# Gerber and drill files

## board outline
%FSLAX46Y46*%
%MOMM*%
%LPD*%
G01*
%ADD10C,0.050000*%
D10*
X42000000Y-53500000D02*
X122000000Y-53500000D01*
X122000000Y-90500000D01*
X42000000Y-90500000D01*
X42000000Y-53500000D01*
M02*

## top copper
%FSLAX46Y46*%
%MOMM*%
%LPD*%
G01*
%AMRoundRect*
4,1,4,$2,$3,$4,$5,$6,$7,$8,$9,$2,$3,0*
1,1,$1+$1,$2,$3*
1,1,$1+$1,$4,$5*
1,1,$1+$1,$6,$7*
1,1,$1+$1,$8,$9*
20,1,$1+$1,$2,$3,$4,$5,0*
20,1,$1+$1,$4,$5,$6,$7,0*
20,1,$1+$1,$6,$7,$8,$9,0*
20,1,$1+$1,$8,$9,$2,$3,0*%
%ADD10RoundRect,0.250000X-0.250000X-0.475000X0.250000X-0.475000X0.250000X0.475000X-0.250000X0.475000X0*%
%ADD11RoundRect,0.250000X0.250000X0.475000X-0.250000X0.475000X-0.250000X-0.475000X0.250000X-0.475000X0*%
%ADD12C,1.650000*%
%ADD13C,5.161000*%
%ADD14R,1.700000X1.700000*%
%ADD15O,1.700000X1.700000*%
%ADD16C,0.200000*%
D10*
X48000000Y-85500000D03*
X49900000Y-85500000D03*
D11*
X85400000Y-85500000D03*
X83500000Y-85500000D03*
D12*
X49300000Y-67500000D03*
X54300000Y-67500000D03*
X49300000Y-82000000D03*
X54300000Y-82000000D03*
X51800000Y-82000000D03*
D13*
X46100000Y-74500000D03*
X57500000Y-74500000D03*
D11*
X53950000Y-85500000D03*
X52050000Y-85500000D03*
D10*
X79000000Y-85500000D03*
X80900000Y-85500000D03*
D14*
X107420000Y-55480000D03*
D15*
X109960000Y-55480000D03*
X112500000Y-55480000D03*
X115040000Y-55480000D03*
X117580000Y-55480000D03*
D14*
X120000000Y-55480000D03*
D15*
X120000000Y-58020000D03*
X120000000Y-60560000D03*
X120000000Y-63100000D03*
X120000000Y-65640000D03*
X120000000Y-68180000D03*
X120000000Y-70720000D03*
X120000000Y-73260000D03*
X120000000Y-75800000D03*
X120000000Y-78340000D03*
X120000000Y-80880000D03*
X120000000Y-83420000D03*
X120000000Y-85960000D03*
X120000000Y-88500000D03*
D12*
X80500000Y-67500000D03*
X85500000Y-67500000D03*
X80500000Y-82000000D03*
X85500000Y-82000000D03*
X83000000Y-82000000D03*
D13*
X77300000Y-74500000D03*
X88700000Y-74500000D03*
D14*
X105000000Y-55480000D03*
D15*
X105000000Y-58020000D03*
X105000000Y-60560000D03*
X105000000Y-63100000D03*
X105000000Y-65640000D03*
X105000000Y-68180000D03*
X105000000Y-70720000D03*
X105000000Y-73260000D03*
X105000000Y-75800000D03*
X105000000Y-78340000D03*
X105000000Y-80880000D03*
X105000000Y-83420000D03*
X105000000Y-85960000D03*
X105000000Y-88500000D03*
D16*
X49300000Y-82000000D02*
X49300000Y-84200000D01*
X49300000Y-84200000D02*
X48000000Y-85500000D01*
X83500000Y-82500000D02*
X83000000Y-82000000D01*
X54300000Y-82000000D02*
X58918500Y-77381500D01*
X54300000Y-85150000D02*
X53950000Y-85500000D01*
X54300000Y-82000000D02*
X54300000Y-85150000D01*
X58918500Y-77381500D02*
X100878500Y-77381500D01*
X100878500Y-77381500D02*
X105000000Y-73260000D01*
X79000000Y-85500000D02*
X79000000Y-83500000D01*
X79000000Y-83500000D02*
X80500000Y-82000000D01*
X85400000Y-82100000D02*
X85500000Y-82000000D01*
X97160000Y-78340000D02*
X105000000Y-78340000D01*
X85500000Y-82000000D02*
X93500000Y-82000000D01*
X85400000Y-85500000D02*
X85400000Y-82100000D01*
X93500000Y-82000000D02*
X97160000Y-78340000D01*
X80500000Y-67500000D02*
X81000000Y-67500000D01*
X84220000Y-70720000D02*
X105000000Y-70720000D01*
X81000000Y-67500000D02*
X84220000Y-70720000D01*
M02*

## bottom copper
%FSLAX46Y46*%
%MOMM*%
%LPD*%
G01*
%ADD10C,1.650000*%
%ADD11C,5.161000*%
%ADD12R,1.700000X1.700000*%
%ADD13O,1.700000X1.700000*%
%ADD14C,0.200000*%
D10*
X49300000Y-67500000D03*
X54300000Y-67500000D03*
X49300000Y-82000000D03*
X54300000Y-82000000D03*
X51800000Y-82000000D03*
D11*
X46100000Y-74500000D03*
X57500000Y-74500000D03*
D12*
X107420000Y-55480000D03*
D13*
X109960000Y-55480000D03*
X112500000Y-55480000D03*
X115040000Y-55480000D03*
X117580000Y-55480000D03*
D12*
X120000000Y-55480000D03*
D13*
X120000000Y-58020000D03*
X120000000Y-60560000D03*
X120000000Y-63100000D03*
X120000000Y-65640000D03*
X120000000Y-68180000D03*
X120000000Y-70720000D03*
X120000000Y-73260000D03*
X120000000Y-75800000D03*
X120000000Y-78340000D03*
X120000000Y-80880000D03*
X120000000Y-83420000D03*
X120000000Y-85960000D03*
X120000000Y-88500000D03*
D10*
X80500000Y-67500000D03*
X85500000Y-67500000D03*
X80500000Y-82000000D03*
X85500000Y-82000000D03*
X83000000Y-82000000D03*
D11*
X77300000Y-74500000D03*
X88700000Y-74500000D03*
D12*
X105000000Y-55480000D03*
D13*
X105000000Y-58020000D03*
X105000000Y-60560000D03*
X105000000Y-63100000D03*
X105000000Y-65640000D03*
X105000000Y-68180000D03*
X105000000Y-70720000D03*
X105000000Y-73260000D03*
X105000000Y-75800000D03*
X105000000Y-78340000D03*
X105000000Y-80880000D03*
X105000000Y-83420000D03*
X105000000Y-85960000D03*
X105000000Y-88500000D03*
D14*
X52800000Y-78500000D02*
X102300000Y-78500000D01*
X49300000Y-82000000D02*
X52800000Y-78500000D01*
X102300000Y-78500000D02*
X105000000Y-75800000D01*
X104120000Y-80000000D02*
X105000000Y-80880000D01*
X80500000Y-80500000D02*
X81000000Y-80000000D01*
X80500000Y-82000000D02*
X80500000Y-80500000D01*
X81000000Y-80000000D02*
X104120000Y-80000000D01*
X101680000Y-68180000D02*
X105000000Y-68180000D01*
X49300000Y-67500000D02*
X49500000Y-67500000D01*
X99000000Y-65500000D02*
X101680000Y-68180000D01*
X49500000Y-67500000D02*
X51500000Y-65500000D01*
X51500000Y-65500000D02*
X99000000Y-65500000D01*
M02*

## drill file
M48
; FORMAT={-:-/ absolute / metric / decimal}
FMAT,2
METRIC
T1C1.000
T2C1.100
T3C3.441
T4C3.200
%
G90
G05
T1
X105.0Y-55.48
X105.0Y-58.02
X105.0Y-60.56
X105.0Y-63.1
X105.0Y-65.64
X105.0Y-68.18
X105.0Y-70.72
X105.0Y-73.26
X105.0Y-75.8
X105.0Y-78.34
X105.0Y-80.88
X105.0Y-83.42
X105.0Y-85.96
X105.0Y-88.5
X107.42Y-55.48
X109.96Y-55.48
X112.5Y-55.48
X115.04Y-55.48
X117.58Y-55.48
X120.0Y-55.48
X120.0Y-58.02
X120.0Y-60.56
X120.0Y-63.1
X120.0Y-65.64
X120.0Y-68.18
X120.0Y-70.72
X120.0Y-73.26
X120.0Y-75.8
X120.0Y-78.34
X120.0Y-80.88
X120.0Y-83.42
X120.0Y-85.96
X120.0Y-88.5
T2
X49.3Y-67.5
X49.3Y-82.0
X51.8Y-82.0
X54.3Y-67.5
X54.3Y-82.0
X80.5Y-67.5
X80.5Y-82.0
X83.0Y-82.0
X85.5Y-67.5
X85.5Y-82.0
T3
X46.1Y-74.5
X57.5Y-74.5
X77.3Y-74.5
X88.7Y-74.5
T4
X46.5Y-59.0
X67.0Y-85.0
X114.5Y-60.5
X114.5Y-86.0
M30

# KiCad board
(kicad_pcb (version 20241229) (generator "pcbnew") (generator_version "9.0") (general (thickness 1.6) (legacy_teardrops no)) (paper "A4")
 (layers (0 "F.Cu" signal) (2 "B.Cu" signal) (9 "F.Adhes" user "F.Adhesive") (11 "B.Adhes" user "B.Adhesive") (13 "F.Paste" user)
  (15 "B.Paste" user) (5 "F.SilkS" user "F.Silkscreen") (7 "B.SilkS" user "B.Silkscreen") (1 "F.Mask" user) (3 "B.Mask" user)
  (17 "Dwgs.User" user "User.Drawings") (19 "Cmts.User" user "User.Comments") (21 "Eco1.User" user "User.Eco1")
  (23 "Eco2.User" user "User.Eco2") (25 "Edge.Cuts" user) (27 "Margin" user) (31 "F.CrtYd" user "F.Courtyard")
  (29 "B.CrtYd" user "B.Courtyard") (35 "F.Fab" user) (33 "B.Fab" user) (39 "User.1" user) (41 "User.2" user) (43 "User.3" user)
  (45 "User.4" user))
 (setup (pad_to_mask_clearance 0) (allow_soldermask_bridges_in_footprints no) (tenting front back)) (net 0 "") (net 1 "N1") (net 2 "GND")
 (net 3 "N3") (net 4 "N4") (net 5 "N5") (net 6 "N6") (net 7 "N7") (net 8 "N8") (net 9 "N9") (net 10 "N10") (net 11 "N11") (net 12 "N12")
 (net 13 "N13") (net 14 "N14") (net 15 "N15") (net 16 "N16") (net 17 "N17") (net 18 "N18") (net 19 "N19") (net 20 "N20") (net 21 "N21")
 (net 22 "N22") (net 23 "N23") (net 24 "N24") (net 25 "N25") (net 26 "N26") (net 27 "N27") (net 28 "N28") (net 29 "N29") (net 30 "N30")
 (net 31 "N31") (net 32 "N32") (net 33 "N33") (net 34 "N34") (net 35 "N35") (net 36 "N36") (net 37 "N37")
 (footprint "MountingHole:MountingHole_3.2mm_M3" (layer "F.Cu") (at 114.5 60.5)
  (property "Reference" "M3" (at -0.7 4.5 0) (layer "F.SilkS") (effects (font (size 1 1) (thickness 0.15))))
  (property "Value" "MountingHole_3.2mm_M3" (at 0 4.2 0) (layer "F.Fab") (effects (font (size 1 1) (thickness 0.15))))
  (pad "" np_thru_hole circle (at 0 0) (size 3.2 3.2) (drill 3.2) (layers "*.Cu" "*.Mask")))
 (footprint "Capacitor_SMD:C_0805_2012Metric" (layer "F.Cu") (at 48.95 85.5)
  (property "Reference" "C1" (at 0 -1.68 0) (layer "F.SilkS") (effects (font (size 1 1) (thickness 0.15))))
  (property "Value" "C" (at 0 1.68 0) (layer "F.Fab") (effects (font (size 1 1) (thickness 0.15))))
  (pad "1" smd roundrect (at -0.95 0) (size 1 1.45) (layers "F.Cu" "F.Mask" "F.Paste") (roundrect_rratio 0.25) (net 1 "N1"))
  (pad "2" smd roundrect (at 0.95 0) (size 1 1.45) (layers "F.Cu" "F.Mask" "F.Paste") (roundrect_rratio 0.25) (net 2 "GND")))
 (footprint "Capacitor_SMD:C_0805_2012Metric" (layer "F.Cu") (at 84.45 85.5 180)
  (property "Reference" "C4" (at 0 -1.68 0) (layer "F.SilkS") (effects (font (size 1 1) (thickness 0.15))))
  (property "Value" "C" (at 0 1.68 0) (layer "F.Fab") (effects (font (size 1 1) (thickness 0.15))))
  (pad "1" smd roundrect (at -0.95 0 180) (size 1 1.45) (layers "F.Cu" "F.Mask" "F.Paste") (roundrect_rratio 0.25) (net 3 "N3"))
  (pad "2" smd roundrect (at 0.95 0 180) (size 1 1.45) (layers "F.Cu" "F.Mask" "F.Paste") (roundrect_rratio 0.25) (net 2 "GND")))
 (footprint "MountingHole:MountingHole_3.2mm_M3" (layer "F.Cu") (at 46.5 59)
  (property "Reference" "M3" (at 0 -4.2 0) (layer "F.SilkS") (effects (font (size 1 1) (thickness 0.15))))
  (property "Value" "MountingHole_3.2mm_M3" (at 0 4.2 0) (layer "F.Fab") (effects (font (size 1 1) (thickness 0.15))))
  (pad "" np_thru_hole circle (at 0 0) (size 3.2 3.2) (drill 3.2) (layers "*.Cu" "*.Mask")))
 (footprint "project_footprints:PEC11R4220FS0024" (layer "F.Cu") (at 49.3 67.5)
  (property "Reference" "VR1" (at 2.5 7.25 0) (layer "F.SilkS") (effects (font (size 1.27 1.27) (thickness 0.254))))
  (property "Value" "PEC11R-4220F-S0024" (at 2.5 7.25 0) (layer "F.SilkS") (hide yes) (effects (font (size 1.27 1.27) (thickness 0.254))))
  (pad "1" thru_hole circle (at 0 0) (size 1.65 1.65) (drill 1.1) (layers "*.Cu" "*.Mask") (remove_unused_layers no) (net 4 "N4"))
  (pad "2" thru_hole circle (at 5 0) (size 1.65 1.65) (drill 1.1) (layers "*.Cu" "*.Mask") (remove_unused_layers no) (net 2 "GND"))
  (pad "A1" thru_hole circle (at 0 14.5) (size 1.65 1.65) (drill 1.1) (layers "*.Cu" "*.Mask") (remove_unused_layers no) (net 1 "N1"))
  (pad "B1" thru_hole circle (at 5 14.5) (size 1.65 1.65) (drill 1.1) (layers "*.Cu" "*.Mask") (remove_unused_layers no) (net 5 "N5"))
  (pad "C1" thru_hole circle (at 2.5 14.5) (size 1.65 1.65) (drill 1.1) (layers "*.Cu" "*.Mask") (remove_unused_layers no) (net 2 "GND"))
  (pad "MH1" thru_hole circle (at -3.2 7) (size 5.161 5.161) (drill 3.4409) (layers "*.Cu" "*.Mask") (remove_unused_layers no) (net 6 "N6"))
  (pad "MH2" thru_hole circle (at 8.2 7) (size 5.161 5.161) (drill 3.4409) (layers "*.Cu" "*.Mask") (remove_unused_layers no) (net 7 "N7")))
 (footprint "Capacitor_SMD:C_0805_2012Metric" (layer "F.Cu") (at 53 85.5 180)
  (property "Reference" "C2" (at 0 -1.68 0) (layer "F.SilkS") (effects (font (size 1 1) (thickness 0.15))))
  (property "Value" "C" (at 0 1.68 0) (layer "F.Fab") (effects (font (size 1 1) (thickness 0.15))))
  (pad "1" smd roundrect (at -0.95 0 180) (size 1 1.45) (layers "F.Cu" "F.Mask" "F.Paste") (roundrect_rratio 0.25) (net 5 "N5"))
  (pad "2" smd roundrect (at 0.95 0 180) (size 1 1.45) (layers "F.Cu" "F.Mask" "F.Paste") (roundrect_rratio 0.25) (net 2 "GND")))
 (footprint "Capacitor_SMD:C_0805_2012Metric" (layer "F.Cu") (at 79.95 85.5)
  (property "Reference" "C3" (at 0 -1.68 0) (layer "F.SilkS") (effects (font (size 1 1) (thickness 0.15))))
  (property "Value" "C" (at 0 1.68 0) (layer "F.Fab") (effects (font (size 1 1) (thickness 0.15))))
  (pad "1" smd roundrect (at -0.95 0) (size 1 1.45) (layers "F.Cu" "F.Mask" "F.Paste") (roundrect_rratio 0.25) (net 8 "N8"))
  (pad "2" smd roundrect (at 0.95 0) (size 1 1.45) (layers "F.Cu" "F.Mask" "F.Paste") (roundrect_rratio 0.25) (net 2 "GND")))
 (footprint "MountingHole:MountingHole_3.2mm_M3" (layer "F.Cu") (at 114.5 86)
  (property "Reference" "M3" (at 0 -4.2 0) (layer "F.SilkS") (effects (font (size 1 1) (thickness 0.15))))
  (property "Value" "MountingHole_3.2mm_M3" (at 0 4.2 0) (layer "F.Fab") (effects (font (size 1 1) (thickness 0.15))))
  (pad "" np_thru_hole circle (at 0 0) (size 3.2 3.2) (drill 3.2) (layers "*.Cu" "*.Mask")))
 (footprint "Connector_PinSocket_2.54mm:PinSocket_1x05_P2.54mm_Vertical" (layer "F.Cu") (at 107.42 55.48 90)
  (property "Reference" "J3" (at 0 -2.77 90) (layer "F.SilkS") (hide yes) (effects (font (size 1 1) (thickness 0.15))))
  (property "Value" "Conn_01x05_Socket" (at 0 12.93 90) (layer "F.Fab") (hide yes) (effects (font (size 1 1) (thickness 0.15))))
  (pad "1" thru_hole rect (at 0 0 90) (size 1.7 1.7) (drill 1) (layers "*.Cu" "*.Mask") (remove_unused_layers no) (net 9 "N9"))
  (pad "2" thru_hole oval (at 0 2.54 90) (size 1.7 1.7) (drill 1) (layers "*.Cu" "*.Mask") (remove_unused_layers no) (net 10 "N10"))
  (pad "3" thru_hole oval (at 0 5.08 90) (size 1.7 1.7) (drill 1) (layers "*.Cu" "*.Mask") (remove_unused_layers no) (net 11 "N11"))
  (pad "4" thru_hole oval (at 0 7.62 90) (size 1.7 1.7) (drill 1) (layers "*.Cu" "*.Mask") (remove_unused_layers no) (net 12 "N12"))
  (pad "5" thru_hole oval (at 0 10.16 90) (size 1.7 1.7) (drill 1) (layers "*.Cu" "*.Mask") (remove_unused_layers no) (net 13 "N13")))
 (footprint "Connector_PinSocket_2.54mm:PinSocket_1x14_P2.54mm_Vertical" (layer "F.Cu") (at 120 55.48)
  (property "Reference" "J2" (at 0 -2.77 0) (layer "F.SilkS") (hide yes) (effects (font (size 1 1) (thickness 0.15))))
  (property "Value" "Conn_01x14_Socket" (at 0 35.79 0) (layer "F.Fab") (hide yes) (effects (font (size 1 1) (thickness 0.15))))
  (pad "1" thru_hole rect (at 0 0) (size 1.7 1.7) (drill 1) (layers "*.Cu" "*.Mask") (remove_unused_layers no) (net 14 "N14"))
  (pad "2" thru_hole oval (at 0 2.54) (size 1.7 1.7) (drill 1) (layers "*.Cu" "*.Mask") (remove_unused_layers no) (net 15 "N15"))
  (pad "3" thru_hole oval (at 0 5.08) (size 1.7 1.7) (drill 1) (layers "*.Cu" "*.Mask") (remove_unused_layers no) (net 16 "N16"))
  (pad "4" thru_hole oval (at 0 7.62) (size 1.7 1.7) (drill 1) (layers "*.Cu" "*.Mask") (remove_unused_layers no) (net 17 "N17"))
  (pad "5" thru_hole oval (at 0 10.16) (size 1.7 1.7) (drill 1) (layers "*.Cu" "*.Mask") (remove_unused_layers no) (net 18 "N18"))
  (pad "6" thru_hole oval (at 0 12.7) (size 1.7 1.7) (drill 1) (layers "*.Cu" "*.Mask") (remove_unused_layers no) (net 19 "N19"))
  (pad "7" thru_hole oval (at 0 15.24) (size 1.7 1.7) (drill 1) (layers "*.Cu" "*.Mask") (remove_unused_layers no) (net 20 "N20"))
  (pad "8" thru_hole oval (at 0 17.78) (size 1.7 1.7) (drill 1) (layers "*.Cu" "*.Mask") (remove_unused_layers no) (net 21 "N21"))
  (pad "9" thru_hole oval (at 0 20.32) (size 1.7 1.7) (drill 1) (layers "*.Cu" "*.Mask") (remove_unused_layers no) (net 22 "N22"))
  (pad "10" thru_hole oval (at 0 22.86) (size 1.7 1.7) (drill 1) (layers "*.Cu" "*.Mask") (remove_unused_layers no) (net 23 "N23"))
  (pad "11" thru_hole oval (at 0 25.4) (size 1.7 1.7) (drill 1) (layers "*.Cu" "*.Mask") (remove_unused_layers no) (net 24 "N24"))
  (pad "12" thru_hole oval (at 0 27.94) (size 1.7 1.7) (drill 1) (layers "*.Cu" "*.Mask") (remove_unused_layers no) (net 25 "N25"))
  (pad "13" thru_hole oval (at 0 30.48) (size 1.7 1.7) (drill 1) (layers "*.Cu" "*.Mask") (remove_unused_layers no) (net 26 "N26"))
  (pad "14" thru_hole oval (at 0 33.02) (size 1.7 1.7) (drill 1) (layers "*.Cu" "*.Mask") (remove_unused_layers no) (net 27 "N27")))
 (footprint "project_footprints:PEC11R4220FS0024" (layer "F.Cu") (at 80.5 67.5)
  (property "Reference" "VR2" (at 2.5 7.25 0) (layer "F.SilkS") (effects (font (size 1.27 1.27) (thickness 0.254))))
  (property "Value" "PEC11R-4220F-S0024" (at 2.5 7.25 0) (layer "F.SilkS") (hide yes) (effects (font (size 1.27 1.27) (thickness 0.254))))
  (pad "1" thru_hole circle (at 0 0) (size 1.65 1.65) (drill 1.1) (layers "*.Cu" "*.Mask") (remove_unused_layers no) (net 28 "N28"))
  (pad "2" thru_hole circle (at 5 0) (size 1.65 1.65) (drill 1.1) (layers "*.Cu" "*.Mask") (remove_unused_layers no) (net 2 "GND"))
  (pad "A1" thru_hole circle (at 0 14.5) (size 1.65 1.65) (drill 1.1) (layers "*.Cu" "*.Mask") (remove_unused_layers no) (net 8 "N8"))
  (pad "B1" thru_hole circle (at 5 14.5) (size 1.65 1.65) (drill 1.1) (layers "*.Cu" "*.Mask") (remove_unused_layers no) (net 3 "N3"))
  (pad "C1" thru_hole circle (at 2.5 14.5) (size 1.65 1.65) (drill 1.1) (layers "*.Cu" "*.Mask") (remove_unused_layers no) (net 2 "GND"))
  (pad "MH1" thru_hole circle (at -3.2 7) (size 5.161 5.161) (drill 3.4409) (layers "*.Cu" "*.Mask") (remove_unused_layers no)
   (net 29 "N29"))
  (pad "MH2" thru_hole circle (at 8.2 7) (size 5.161 5.161) (drill 3.4409) (layers "*.Cu" "*.Mask") (remove_unused_layers no) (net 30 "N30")))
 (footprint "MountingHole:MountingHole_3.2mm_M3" (layer "F.Cu") (at 67 85)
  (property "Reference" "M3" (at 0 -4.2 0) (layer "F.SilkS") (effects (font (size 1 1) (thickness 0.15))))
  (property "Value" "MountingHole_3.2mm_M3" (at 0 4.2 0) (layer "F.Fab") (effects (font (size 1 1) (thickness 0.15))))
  (pad "" np_thru_hole circle (at 0 0) (size 3.2 3.2) (drill 3.2) (layers "*.Cu" "*.Mask")))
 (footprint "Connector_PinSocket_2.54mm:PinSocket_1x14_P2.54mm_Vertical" (layer "F.Cu") (at 105 55.48)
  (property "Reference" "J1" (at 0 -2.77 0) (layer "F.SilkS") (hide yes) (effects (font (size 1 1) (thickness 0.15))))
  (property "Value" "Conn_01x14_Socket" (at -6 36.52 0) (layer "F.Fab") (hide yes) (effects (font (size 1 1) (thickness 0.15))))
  (pad "1" thru_hole rect (at 0 0) (size 1.7 1.7) (drill 1) (layers "*.Cu" "*.Mask") (remove_unused_layers no) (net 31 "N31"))
  (pad "2" thru_hole oval (at 0 2.54) (size 1.7 1.7) (drill 1) (layers "*.Cu" "*.Mask") (remove_unused_layers no) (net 2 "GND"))
  (pad "3" thru_hole oval (at 0 5.08) (size 1.7 1.7) (drill 1) (layers "*.Cu" "*.Mask") (remove_unused_layers no) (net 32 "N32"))
  (pad "4" thru_hole oval (at 0 7.62) (size 1.7 1.7) (drill 1) (layers "*.Cu" "*.Mask") (remove_unused_layers no) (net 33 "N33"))
  (pad "5" thru_hole oval (at 0 10.16) (size 1.7 1.7) (drill 1) (layers "*.Cu" "*.Mask") (remove_unused_layers no) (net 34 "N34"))
  (pad "6" thru_hole oval (at 0 12.7) (size 1.7 1.7) (drill 1) (layers "*.Cu" "*.Mask") (remove_unused_layers no) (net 4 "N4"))
  (pad "7" thru_hole oval (at 0 15.24) (size 1.7 1.7) (drill 1) (layers "*.Cu" "*.Mask") (remove_unused_layers no) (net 28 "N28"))
  (pad "8" thru_hole oval (at 0 17.78) (size 1.7 1.7) (drill 1) (layers "*.Cu" "*.Mask") (remove_unused_layers no) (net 5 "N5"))
  (pad "9" thru_hole oval (at 0 20.32) (size 1.7 1.7) (drill 1) (layers "*.Cu" "*.Mask") (remove_unused_layers no) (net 1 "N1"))
  (pad "10" thru_hole oval (at 0 22.86) (size 1.7 1.7) (drill 1) (layers "*.Cu" "*.Mask") (remove_unused_layers no) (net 3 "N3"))
  (pad "11" thru_hole oval (at 0 25.4) (size 1.7 1.7) (drill 1) (layers "*.Cu" "*.Mask") (remove_unused_layers no) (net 8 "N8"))
  (pad "12" thru_hole oval (at 0 27.94) (size 1.7 1.7) (drill 1) (layers "*.Cu" "*.Mask") (remove_unused_layers no) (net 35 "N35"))
  (pad "13" thru_hole oval (at 0 30.48) (size 1.7 1.7) (drill 1) (layers "*.Cu" "*.Mask") (remove_unused_layers no) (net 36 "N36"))
  (pad "14" thru_hole oval (at 0 33.02) (size 1.7 1.7) (drill 1) (layers "*.Cu" "*.Mask") (remove_unused_layers no) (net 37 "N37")))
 (gr_rect (start 42 53.5) (end 122 90.5) (stroke (width 0.05) (type default)) (fill no) (layer "Edge.Cuts"))
 (segment (start 49.3 82) (end 49.3 84.2) (width 0.2) (layer "F.Cu") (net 1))
 (segment (start 49.3 84.2) (end 48 85.5) (width 0.2) (layer "F.Cu") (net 1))
 (segment (start 52.8 78.5) (end 102.3 78.5) (width 0.2) (layer "B.Cu") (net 1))
 (segment (start 49.3 82) (end 52.8 78.5) (width 0.2) (layer "B.Cu") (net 1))
 (segment (start 102.3 78.5) (end 105 75.8) (width 0.2) (layer "B.Cu") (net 1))
 (segment (start 83.5 82.5) (end 83 82) (width 0.2) (layer "F.Cu") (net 2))
 (segment (start 54.3 82) (end 58.9185 77.3815) (width 0.2) (layer "F.Cu") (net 5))
 (segment (start 54.3 85.15) (end 53.95 85.5) (width 0.2) (layer "F.Cu") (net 5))
 (segment (start 54.3 82) (end 54.3 85.15) (width 0.2) (layer "F.Cu") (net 5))
 (segment (start 58.9185 77.3815) (end 100.8785 77.3815) (width 0.2) (layer "F.Cu") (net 5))
 (segment (start 100.8785 77.3815) (end 105 73.26) (width 0.2) (layer "F.Cu") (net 5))
 (segment (start 79 85.5) (end 79 83.5) (width 0.2) (layer "F.Cu") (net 8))
 (segment (start 79 83.5) (end 80.5 82) (width 0.2) (layer "F.Cu") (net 8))
 (segment (start 104.12 80) (end 105 80.88) (width 0.2) (layer "B.Cu") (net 8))
 (segment (start 80.5 80.5) (end 81 80) (width 0.2) (layer "B.Cu") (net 8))
 (segment (start 80.5 82) (end 80.5 80.5) (width 0.2) (layer "B.Cu") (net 8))
 (segment (start 81 80) (end 104.12 80) (width 0.2) (layer "B.Cu") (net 8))
 (segment (start 85.4 82.1) (end 85.5 82) (width 0.2) (layer "F.Cu") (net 3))
 (segment (start 97.16 78.34) (end 105 78.34) (width 0.2) (layer "F.Cu") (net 3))
 (segment (start 85.5 82) (end 93.5 82) (width 0.2) (layer "F.Cu") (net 3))
 (segment (start 85.4 85.5) (end 85.4 82.1) (width 0.2) (layer "F.Cu") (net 3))
 (segment (start 93.5 82) (end 97.16 78.34) (width 0.2) (layer "F.Cu") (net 3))
 (segment (start 80.5 67.5) (end 81 67.5) (width 0.2) (layer "F.Cu") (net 28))
 (segment (start 84.22 70.72) (end 105 70.72) (width 0.2) (layer "F.Cu") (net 28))
 (segment (start 81 67.5) (end 84.22 70.72) (width 0.2) (layer "F.Cu") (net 28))
 (segment (start 101.68 68.18) (end 105 68.18) (width 0.2) (layer "B.Cu") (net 4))
 (segment (start 49.3 67.5) (end 49.5 67.5) (width 0.2) (layer "B.Cu") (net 4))
 (segment (start 99 65.5) (end 101.68 68.18) (width 0.2) (layer "B.Cu") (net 4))
 (segment (start 49.5 67.5) (end 51.5 65.5) (width 0.2) (layer "B.Cu") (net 4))
 (segment (start 51.5 65.5) (end 99 65.5) (width 0.2) (layer "B.Cu") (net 4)))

